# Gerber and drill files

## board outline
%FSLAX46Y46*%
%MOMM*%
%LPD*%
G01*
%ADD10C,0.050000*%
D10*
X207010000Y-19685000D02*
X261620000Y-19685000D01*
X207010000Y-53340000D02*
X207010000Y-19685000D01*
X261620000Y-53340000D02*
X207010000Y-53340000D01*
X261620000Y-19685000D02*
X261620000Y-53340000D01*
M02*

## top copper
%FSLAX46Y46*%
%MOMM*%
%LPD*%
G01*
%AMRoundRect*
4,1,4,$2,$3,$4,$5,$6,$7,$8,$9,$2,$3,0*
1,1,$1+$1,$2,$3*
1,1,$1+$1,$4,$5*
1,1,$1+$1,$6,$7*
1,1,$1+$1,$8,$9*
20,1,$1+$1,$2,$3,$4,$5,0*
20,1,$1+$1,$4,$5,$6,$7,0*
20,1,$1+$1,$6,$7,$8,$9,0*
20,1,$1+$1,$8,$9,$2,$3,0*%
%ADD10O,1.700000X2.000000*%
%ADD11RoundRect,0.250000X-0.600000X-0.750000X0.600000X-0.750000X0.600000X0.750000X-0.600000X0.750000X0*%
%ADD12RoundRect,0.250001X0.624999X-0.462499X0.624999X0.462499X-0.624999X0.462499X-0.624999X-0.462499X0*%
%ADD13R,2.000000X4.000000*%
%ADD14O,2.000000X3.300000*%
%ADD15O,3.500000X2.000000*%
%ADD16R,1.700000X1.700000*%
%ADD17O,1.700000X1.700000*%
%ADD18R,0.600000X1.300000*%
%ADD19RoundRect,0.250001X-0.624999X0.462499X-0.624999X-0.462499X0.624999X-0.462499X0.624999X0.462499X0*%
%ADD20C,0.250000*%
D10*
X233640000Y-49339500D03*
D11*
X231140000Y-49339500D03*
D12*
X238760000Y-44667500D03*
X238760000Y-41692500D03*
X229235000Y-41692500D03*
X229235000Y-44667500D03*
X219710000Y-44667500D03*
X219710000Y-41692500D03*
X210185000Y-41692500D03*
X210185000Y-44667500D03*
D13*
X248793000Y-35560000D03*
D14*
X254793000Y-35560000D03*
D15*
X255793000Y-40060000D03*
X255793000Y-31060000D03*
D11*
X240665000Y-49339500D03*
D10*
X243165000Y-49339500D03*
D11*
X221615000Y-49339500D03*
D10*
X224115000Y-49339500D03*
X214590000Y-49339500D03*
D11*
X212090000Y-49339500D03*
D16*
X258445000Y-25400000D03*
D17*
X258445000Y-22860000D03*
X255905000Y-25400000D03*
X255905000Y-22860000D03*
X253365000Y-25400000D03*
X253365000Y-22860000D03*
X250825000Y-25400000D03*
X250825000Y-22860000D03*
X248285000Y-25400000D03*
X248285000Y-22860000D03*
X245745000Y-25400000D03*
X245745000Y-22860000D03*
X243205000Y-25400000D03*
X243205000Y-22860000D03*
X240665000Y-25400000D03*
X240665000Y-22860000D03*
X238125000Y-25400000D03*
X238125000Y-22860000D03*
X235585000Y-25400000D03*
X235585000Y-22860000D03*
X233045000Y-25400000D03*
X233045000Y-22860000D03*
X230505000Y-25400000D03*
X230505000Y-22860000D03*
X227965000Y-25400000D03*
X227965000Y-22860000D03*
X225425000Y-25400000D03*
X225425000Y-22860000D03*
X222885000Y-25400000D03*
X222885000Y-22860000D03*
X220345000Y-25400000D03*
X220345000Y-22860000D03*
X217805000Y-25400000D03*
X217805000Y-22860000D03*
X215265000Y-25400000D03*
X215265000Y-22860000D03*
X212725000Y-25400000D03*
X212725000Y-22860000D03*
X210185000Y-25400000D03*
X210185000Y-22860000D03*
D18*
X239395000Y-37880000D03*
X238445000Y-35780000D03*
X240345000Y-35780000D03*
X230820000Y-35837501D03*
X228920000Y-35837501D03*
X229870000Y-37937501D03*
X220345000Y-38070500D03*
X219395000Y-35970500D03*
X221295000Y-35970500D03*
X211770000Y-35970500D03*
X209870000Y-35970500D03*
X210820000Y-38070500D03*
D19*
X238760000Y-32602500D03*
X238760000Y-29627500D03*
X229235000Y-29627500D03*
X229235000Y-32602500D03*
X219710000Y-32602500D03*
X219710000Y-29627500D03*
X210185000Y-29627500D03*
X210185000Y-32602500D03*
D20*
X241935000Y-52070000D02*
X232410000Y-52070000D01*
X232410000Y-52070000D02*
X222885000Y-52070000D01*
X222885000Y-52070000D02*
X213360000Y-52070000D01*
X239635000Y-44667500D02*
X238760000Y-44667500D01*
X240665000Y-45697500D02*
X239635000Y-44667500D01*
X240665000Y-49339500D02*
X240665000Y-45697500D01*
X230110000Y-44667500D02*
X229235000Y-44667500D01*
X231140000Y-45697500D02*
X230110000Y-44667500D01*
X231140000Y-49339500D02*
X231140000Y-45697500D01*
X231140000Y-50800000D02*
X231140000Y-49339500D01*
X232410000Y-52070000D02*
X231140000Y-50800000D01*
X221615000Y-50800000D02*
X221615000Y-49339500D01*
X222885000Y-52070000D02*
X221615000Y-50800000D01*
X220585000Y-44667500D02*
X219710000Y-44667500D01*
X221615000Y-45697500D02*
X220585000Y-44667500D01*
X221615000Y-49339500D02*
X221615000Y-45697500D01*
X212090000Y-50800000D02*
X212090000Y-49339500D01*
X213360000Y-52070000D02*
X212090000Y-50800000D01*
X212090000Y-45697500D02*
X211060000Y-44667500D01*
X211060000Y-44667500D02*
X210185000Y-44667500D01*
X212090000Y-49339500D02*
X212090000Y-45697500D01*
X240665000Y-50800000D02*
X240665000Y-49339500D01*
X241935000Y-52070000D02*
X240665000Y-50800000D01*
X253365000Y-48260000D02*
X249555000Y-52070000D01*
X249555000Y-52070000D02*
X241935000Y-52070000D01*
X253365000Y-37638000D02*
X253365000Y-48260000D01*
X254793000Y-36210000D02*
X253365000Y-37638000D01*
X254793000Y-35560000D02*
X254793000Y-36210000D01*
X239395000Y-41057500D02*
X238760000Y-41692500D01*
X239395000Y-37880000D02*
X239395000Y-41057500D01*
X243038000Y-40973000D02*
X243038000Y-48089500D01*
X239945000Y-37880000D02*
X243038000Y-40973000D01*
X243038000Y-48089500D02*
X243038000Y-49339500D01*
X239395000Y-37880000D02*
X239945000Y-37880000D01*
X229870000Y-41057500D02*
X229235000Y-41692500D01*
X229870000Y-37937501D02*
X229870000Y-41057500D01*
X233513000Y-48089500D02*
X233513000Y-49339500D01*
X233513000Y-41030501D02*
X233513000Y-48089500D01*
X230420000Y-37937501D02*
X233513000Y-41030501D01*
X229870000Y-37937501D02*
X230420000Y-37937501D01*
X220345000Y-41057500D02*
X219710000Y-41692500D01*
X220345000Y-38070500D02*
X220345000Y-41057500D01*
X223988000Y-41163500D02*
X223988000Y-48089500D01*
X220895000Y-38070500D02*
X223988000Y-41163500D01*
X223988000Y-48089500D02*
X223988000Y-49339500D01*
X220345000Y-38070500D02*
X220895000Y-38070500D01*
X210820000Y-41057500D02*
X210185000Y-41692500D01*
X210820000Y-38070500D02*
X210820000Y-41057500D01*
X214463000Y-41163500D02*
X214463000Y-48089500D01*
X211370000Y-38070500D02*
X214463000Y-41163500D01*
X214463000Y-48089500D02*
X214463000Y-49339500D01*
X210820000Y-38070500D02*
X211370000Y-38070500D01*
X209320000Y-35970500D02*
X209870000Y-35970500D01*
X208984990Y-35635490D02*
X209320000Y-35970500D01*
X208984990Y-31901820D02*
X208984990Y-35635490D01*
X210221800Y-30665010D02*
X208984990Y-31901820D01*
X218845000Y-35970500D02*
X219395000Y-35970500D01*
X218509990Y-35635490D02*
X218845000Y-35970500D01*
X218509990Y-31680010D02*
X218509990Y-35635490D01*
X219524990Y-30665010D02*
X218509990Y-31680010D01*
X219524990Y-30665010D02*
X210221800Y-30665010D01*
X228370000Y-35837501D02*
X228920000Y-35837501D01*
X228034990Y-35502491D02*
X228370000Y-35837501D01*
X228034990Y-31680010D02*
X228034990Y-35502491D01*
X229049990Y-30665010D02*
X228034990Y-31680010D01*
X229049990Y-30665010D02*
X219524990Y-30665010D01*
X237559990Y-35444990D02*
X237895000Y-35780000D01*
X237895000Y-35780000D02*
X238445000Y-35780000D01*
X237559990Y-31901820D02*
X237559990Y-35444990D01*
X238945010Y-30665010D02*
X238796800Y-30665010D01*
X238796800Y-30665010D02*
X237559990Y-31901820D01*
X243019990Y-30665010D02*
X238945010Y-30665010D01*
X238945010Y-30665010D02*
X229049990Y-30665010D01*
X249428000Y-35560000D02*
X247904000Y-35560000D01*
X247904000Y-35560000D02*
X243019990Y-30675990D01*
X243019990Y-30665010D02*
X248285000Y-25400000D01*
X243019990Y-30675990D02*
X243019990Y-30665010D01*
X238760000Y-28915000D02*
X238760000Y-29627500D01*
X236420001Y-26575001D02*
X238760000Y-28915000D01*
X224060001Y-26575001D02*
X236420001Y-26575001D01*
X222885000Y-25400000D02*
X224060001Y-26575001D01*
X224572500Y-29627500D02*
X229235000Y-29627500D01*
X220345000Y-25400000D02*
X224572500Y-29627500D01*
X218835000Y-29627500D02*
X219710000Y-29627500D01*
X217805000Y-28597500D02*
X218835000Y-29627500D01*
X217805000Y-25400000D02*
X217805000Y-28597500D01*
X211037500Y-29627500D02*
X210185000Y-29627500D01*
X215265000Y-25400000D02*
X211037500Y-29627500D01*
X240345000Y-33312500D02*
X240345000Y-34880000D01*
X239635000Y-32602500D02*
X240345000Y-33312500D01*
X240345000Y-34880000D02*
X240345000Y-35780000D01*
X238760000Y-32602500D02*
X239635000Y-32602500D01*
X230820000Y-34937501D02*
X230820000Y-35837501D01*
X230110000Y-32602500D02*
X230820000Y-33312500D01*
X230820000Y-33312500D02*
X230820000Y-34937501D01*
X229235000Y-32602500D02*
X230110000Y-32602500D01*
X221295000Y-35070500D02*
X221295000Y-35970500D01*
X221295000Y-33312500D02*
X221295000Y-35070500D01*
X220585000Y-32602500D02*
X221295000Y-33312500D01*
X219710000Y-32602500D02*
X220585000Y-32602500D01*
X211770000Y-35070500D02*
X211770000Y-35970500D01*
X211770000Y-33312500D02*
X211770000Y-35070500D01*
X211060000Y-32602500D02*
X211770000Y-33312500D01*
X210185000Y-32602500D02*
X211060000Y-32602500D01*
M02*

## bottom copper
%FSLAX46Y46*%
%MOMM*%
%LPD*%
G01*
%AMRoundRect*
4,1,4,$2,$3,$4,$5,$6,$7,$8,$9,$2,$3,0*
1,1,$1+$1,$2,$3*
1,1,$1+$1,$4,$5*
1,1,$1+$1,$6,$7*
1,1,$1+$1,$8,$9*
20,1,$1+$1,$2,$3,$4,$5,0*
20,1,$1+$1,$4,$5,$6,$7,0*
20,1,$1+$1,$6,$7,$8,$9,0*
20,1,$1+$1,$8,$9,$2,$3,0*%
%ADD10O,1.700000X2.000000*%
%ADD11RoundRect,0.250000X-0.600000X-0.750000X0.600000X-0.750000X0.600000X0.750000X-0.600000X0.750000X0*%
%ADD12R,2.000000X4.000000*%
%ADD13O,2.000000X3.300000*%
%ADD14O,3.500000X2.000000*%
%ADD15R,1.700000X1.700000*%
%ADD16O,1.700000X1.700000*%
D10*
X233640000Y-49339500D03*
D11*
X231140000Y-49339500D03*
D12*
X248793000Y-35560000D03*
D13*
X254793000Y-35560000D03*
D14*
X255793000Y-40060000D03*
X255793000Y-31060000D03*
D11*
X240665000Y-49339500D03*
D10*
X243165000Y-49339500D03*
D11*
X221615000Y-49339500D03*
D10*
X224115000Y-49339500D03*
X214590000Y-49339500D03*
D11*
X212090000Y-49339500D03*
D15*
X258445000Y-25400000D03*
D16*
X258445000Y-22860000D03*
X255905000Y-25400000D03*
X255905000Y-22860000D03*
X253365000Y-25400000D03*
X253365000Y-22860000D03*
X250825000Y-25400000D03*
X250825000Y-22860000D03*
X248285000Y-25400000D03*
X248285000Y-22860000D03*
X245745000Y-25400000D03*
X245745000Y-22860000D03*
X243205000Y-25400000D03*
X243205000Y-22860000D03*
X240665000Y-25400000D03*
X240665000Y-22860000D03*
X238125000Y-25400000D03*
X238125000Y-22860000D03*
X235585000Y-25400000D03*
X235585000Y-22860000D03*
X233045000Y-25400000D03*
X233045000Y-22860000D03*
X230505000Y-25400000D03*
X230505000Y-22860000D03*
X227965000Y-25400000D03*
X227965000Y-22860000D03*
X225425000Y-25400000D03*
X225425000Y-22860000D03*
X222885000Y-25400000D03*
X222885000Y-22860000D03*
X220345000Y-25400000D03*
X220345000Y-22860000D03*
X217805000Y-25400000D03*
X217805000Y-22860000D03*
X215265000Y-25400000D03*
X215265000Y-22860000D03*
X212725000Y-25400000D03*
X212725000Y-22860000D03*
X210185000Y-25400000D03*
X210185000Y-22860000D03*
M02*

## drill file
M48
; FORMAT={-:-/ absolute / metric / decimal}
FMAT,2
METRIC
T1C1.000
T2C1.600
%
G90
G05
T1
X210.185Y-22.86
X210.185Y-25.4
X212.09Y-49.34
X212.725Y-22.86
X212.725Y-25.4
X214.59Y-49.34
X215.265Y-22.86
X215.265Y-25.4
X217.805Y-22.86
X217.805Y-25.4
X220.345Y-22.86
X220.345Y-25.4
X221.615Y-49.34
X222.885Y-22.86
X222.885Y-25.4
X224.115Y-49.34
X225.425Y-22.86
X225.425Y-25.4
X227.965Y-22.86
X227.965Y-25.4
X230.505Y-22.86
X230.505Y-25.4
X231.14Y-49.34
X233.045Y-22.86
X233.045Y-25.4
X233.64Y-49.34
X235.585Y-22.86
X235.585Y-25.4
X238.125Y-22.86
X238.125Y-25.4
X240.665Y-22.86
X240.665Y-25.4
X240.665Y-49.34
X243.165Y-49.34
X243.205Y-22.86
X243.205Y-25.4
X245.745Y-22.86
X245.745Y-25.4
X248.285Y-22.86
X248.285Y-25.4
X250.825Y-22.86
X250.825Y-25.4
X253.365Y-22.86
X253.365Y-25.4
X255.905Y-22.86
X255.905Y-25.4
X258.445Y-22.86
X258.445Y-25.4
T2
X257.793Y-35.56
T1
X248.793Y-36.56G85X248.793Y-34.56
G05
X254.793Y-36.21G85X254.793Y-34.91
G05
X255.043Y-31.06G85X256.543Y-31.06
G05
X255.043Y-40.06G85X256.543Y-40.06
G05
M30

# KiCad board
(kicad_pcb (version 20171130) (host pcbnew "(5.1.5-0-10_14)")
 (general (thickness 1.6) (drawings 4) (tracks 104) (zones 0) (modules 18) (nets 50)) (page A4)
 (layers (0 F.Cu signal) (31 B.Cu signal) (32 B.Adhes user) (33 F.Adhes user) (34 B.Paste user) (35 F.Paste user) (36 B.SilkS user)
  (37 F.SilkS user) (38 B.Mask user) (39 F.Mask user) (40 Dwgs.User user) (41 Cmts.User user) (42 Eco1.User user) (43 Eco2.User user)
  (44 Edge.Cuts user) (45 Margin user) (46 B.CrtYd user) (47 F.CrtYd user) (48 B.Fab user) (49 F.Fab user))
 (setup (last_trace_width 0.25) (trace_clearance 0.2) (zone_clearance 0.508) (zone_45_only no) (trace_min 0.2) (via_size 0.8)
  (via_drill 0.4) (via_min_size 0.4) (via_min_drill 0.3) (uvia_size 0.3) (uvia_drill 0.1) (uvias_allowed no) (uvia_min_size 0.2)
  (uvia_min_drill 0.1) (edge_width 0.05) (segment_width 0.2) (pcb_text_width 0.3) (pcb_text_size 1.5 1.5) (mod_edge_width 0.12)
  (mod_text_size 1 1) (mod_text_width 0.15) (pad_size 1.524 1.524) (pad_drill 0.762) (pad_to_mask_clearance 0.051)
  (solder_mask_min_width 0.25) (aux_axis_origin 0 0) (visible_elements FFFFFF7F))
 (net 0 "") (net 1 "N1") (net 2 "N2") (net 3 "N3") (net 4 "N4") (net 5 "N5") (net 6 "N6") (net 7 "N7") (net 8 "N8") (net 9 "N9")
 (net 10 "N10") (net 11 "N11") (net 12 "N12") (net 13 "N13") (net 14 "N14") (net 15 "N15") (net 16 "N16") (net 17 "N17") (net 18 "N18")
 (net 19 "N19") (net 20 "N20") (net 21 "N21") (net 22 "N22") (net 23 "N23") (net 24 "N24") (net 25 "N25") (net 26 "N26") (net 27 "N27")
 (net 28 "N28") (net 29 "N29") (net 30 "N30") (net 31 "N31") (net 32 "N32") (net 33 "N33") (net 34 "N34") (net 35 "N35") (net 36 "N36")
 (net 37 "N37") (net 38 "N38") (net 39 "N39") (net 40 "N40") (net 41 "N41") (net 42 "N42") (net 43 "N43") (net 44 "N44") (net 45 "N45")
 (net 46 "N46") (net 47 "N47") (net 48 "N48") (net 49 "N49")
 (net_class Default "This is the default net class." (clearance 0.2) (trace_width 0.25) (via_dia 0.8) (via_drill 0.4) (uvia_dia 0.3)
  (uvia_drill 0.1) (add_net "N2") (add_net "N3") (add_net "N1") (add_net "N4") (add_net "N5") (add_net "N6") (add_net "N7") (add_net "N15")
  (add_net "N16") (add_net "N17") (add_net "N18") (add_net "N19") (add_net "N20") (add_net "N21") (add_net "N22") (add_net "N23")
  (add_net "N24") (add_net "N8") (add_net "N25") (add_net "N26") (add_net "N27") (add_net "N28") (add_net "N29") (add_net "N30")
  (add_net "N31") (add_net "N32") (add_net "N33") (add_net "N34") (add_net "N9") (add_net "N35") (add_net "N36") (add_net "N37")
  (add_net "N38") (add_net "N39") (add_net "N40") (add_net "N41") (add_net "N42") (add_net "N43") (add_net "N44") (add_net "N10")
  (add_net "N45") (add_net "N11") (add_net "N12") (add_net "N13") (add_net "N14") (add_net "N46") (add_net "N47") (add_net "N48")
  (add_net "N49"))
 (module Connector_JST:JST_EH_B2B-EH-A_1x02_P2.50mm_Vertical (layer F.Cu) (at 231.14 49.3395)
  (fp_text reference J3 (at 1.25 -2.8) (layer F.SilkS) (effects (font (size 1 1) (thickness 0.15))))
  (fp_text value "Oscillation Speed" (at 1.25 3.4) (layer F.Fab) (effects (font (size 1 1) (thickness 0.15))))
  (pad 2 thru_hole oval (at 2.5 0) (size 1.7 2) (drill 1) (layers *.Cu *.Mask) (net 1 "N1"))
  (pad 1 thru_hole roundrect (at 0 0) (size 1.7 2) (drill 1) (layers *.Cu *.Mask) (roundrect_rratio 0.147059) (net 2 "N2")))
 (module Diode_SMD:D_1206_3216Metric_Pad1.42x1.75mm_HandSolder (layer F.Cu) (at 238.76 43.18 90)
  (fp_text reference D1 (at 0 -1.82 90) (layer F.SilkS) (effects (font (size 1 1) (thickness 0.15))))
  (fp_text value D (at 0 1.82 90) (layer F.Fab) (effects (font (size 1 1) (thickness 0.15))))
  (pad 1 smd roundrect (at -1.4875 0 90) (size 1.425 1.75) (layers F.Cu F.Paste F.Mask) (roundrect_rratio 0.175439) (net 2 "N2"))
  (pad 2 smd roundrect (at 1.4875 0 90) (size 1.425 1.75) (layers F.Cu F.Paste F.Mask) (roundrect_rratio 0.175439) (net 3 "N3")))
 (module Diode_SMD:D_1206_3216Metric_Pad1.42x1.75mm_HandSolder (layer F.Cu) (at 229.235 43.18 90)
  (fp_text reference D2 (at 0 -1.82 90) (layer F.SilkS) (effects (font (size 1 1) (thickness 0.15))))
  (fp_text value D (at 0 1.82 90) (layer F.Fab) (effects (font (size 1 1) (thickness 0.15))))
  (pad 2 smd roundrect (at 1.4875 0 90) (size 1.425 1.75) (layers F.Cu F.Paste F.Mask) (roundrect_rratio 0.175439) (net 1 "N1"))
  (pad 1 smd roundrect (at -1.4875 0 90) (size 1.425 1.75) (layers F.Cu F.Paste F.Mask) (roundrect_rratio 0.175439) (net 2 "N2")))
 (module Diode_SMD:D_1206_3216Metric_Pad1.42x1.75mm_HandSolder (layer F.Cu) (at 219.71 43.18 90)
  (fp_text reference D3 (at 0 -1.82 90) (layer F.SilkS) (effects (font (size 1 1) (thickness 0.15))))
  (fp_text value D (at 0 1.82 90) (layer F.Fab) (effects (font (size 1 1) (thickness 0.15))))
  (pad 1 smd roundrect (at -1.4875 0 90) (size 1.425 1.75) (layers F.Cu F.Paste F.Mask) (roundrect_rratio 0.175439) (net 2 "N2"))
  (pad 2 smd roundrect (at 1.4875 0 90) (size 1.425 1.75) (layers F.Cu F.Paste F.Mask) (roundrect_rratio 0.175439) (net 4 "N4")))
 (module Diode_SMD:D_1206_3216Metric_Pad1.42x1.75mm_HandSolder (layer F.Cu) (at 210.185 43.18 90)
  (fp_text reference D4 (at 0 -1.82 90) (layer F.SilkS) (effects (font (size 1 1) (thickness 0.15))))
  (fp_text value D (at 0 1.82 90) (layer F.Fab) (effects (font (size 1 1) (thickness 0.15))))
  (pad 2 smd roundrect (at 1.4875 0 90) (size 1.425 1.75) (layers F.Cu F.Paste F.Mask) (roundrect_rratio 0.175439) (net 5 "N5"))
  (pad 1 smd roundrect (at -1.4875 0 90) (size 1.425 1.75) (layers F.Cu F.Paste F.Mask) (roundrect_rratio 0.175439) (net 2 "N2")))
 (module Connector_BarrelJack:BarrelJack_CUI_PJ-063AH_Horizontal (layer F.Cu) (at 248.793 35.56 90)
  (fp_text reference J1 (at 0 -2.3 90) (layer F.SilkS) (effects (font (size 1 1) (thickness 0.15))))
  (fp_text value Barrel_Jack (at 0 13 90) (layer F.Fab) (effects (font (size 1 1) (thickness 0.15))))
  (pad 1 thru_hole rect (at 0 0 90) (size 4 2) (drill oval 3 1) (layers *.Cu *.Mask) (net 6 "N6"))
  (pad 2 thru_hole oval (at 0 6 90) (size 3.3 2) (drill oval 2.3 1) (layers *.Cu *.Mask) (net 2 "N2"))
  (pad MP thru_hole oval (at -4.5 7 90) (size 2 3.5) (drill oval 1 2.5) (layers *.Cu *.Mask))
  (pad MP thru_hole oval (at 4.5 7 90) (size 2 3.5) (drill oval 1 2.5) (layers *.Cu *.Mask))
  (pad "" np_thru_hole circle (at 0 9 90) (size 1.6 1.6) (drill 1.6) (layers *.Cu *.Mask)))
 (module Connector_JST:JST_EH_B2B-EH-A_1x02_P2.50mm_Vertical (layer F.Cu) (at 240.665 49.3395)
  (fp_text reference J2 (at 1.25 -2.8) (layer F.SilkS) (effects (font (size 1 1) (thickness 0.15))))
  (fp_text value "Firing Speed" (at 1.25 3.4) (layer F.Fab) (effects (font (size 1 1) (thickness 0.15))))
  (pad 1 thru_hole roundrect (at 0 0) (size 1.7 2) (drill 1) (layers *.Cu *.Mask) (roundrect_rratio 0.147059) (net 2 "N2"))
  (pad 2 thru_hole oval (at 2.5 0) (size 1.7 2) (drill 1) (layers *.Cu *.Mask) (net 3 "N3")))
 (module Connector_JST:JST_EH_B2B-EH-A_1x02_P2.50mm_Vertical (layer F.Cu) (at 221.615 49.3395)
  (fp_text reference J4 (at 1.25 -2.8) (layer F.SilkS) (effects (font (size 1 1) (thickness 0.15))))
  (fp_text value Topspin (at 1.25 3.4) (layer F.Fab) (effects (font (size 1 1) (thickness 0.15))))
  (pad 1 thru_hole roundrect (at 0 0) (size 1.7 2) (drill 1) (layers *.Cu *.Mask) (roundrect_rratio 0.147059) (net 2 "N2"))
  (pad 2 thru_hole oval (at 2.5 0) (size 1.7 2) (drill 1) (layers *.Cu *.Mask) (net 4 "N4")))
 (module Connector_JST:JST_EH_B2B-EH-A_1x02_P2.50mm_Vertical (layer F.Cu) (at 212.09 49.3395)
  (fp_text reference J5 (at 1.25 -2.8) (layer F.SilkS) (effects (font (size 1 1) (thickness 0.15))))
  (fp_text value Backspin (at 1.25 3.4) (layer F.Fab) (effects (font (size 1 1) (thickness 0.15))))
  (pad 2 thru_hole oval (at 2.5 0) (size 1.7 2) (drill 1) (layers *.Cu *.Mask) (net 5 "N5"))
  (pad 1 thru_hole roundrect (at 0 0) (size 1.7 2) (drill 1) (layers *.Cu *.Mask) (roundrect_rratio 0.147059) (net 2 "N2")))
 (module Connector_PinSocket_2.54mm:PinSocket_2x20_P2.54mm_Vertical (layer F.Cu) (at 258.445 25.4 270)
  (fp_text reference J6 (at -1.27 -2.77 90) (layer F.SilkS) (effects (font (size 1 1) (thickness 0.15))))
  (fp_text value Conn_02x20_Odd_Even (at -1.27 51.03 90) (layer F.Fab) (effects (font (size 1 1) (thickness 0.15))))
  (pad 1 thru_hole rect (at 0 0 270) (size 1.7 1.7) (drill 1) (layers *.Cu *.Mask) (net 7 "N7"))
  (pad 2 thru_hole oval (at -2.54 0 270) (size 1.7 1.7) (drill 1) (layers *.Cu *.Mask) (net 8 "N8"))
  (pad 3 thru_hole oval (at 0 2.54 270) (size 1.7 1.7) (drill 1) (layers *.Cu *.Mask) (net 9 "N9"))
  (pad 4 thru_hole oval (at -2.54 2.54 270) (size 1.7 1.7) (drill 1) (layers *.Cu *.Mask) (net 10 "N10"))
  (pad 5 thru_hole oval (at 0 5.08 270) (size 1.7 1.7) (drill 1) (layers *.Cu *.Mask) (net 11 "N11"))
  (pad 6 thru_hole oval (at -2.54 5.08 270) (size 1.7 1.7) (drill 1) (layers *.Cu *.Mask) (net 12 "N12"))
  (pad 7 thru_hole oval (at 0 7.62 270) (size 1.7 1.7) (drill 1) (layers *.Cu *.Mask) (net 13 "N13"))
  (pad 8 thru_hole oval (at -2.54 7.62 270) (size 1.7 1.7) (drill 1) (layers *.Cu *.Mask) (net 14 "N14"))
  (pad 9 thru_hole oval (at 0 10.16 270) (size 1.7 1.7) (drill 1) (layers *.Cu *.Mask) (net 6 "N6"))
  (pad 10 thru_hole oval (at -2.54 10.16 270) (size 1.7 1.7) (drill 1) (layers *.Cu *.Mask) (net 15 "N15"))
  (pad 11 thru_hole oval (at 0 12.7 270) (size 1.7 1.7) (drill 1) (layers *.Cu *.Mask) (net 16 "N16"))
  (pad 12 thru_hole oval (at -2.54 12.7 270) (size 1.7 1.7) (drill 1) (layers *.Cu *.Mask) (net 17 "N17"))
  (pad 13 thru_hole oval (at 0 15.24 270) (size 1.7 1.7) (drill 1) (layers *.Cu *.Mask) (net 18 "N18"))
  (pad 14 thru_hole oval (at -2.54 15.24 270) (size 1.7 1.7) (drill 1) (layers *.Cu *.Mask) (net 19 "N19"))
  (pad 15 thru_hole oval (at 0 17.78 270) (size 1.7 1.7) (drill 1) (layers *.Cu *.Mask) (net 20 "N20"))
  (pad 16 thru_hole oval (at -2.54 17.78 270) (size 1.7 1.7) (drill 1) (layers *.Cu *.Mask) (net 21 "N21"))
  (pad 17 thru_hole oval (at 0 20.32 270) (size 1.7 1.7) (drill 1) (layers *.Cu *.Mask) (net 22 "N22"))
  (pad 18 thru_hole oval (at -2.54 20.32 270) (size 1.7 1.7) (drill 1) (layers *.Cu *.Mask) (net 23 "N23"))
  (pad 19 thru_hole oval (at 0 22.86 270) (size 1.7 1.7) (drill 1) (layers *.Cu *.Mask) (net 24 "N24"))
  (pad 20 thru_hole oval (at -2.54 22.86 270) (size 1.7 1.7) (drill 1) (layers *.Cu *.Mask) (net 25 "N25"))
  (pad 21 thru_hole oval (at 0 25.4 270) (size 1.7 1.7) (drill 1) (layers *.Cu *.Mask) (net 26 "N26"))
  (pad 22 thru_hole oval (at -2.54 25.4 270) (size 1.7 1.7) (drill 1) (layers *.Cu *.Mask) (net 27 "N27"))
  (pad 23 thru_hole oval (at 0 27.94 270) (size 1.7 1.7) (drill 1) (layers *.Cu *.Mask) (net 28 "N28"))
  (pad 24 thru_hole oval (at -2.54 27.94 270) (size 1.7 1.7) (drill 1) (layers *.Cu *.Mask) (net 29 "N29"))
  (pad 25 thru_hole oval (at 0 30.48 270) (size 1.7 1.7) (drill 1) (layers *.Cu *.Mask) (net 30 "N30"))
  (pad 26 thru_hole oval (at -2.54 30.48 270) (size 1.7 1.7) (drill 1) (layers *.Cu *.Mask) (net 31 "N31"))
  (pad 27 thru_hole oval (at 0 33.02 270) (size 1.7 1.7) (drill 1) (layers *.Cu *.Mask) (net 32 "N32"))
  (pad 28 thru_hole oval (at -2.54 33.02 270) (size 1.7 1.7) (drill 1) (layers *.Cu *.Mask) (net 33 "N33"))
  (pad 29 thru_hole oval (at 0 35.56 270) (size 1.7 1.7) (drill 1) (layers *.Cu *.Mask) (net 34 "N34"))
  (pad 30 thru_hole oval (at -2.54 35.56 270) (size 1.7 1.7) (drill 1) (layers *.Cu *.Mask) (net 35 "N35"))
  (pad 31 thru_hole oval (at 0 38.1 270) (size 1.7 1.7) (drill 1) (layers *.Cu *.Mask) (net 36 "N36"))
  (pad 32 thru_hole oval (at -2.54 38.1 270) (size 1.7 1.7) (drill 1) (layers *.Cu *.Mask) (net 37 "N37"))
  (pad 33 thru_hole oval (at 0 40.64 270) (size 1.7 1.7) (drill 1) (layers *.Cu *.Mask) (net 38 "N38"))
  (pad 34 thru_hole oval (at -2.54 40.64 270) (size 1.7 1.7) (drill 1) (layers *.Cu *.Mask) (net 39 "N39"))
  (pad 35 thru_hole oval (at 0 43.18 270) (size 1.7 1.7) (drill 1) (layers *.Cu *.Mask) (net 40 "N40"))
  (pad 36 thru_hole oval (at -2.54 43.18 270) (size 1.7 1.7) (drill 1) (layers *.Cu *.Mask) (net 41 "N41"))
  (pad 37 thru_hole oval (at 0 45.72 270) (size 1.7 1.7) (drill 1) (layers *.Cu *.Mask) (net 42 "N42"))
  (pad 38 thru_hole oval (at -2.54 45.72 270) (size 1.7 1.7) (drill 1) (layers *.Cu *.Mask) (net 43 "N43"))
  (pad 39 thru_hole oval (at 0 48.26 270) (size 1.7 1.7) (drill 1) (layers *.Cu *.Mask) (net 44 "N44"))
  (pad 40 thru_hole oval (at -2.54 48.26 270) (size 1.7 1.7) (drill 1) (layers *.Cu *.Mask) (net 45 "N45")))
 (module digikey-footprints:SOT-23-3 (layer F.Cu) (at 239.395 36.83 270)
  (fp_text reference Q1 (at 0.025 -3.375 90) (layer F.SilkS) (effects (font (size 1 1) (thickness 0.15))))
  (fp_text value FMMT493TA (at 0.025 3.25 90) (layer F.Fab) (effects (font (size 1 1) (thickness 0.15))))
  (pad 3 smd rect (at 1.05 0 270) (size 1.3 0.6) (layers F.Cu F.Paste F.Mask) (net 3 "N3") (solder_mask_margin 0.07))
  (pad 2 smd rect (at -1.05 0.95 270) (size 1.3 0.6) (layers F.Cu F.Paste F.Mask) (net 6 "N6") (solder_mask_margin 0.07))
  (pad 1 smd rect (at -1.05 -0.95 270) (size 1.3 0.6) (layers F.Cu F.Paste F.Mask) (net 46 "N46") (solder_mask_margin 0.07)))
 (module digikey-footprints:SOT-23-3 (layer F.Cu) (at 229.87 36.887501 270)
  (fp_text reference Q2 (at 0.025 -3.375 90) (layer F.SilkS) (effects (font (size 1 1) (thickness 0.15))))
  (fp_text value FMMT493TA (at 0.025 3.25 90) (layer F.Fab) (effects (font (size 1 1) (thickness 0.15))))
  (pad 1 smd rect (at -1.05 -0.95 270) (size 1.3 0.6) (layers F.Cu F.Paste F.Mask) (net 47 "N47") (solder_mask_margin 0.07))
  (pad 2 smd rect (at -1.05 0.95 270) (size 1.3 0.6) (layers F.Cu F.Paste F.Mask) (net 6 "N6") (solder_mask_margin 0.07))
  (pad 3 smd rect (at 1.05 0 270) (size 1.3 0.6) (layers F.Cu F.Paste F.Mask) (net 1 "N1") (solder_mask_margin 0.07)))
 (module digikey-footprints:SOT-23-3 (layer F.Cu) (at 220.345 37.0205 270)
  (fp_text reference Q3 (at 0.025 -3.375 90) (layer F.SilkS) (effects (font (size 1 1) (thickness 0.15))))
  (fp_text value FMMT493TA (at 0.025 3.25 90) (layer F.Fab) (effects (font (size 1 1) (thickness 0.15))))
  (pad 3 smd rect (at 1.05 0 270) (size 1.3 0.6) (layers F.Cu F.Paste F.Mask) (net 4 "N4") (solder_mask_margin 0.07))
  (pad 2 smd rect (at -1.05 0.95 270) (size 1.3 0.6) (layers F.Cu F.Paste F.Mask) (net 6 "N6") (solder_mask_margin 0.07))
  (pad 1 smd rect (at -1.05 -0.95 270) (size 1.3 0.6) (layers F.Cu F.Paste F.Mask) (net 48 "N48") (solder_mask_margin 0.07)))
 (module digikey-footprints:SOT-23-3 (layer F.Cu) (at 210.82 37.0205 270)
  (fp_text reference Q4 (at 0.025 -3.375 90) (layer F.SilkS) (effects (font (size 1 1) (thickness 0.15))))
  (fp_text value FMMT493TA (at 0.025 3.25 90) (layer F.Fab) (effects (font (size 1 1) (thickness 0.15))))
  (pad 1 smd rect (at -1.05 -0.95 270) (size 1.3 0.6) (layers F.Cu F.Paste F.Mask) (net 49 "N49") (solder_mask_margin 0.07))
  (pad 2 smd rect (at -1.05 0.95 270) (size 1.3 0.6) (layers F.Cu F.Paste F.Mask) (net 6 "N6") (solder_mask_margin 0.07))
  (pad 3 smd rect (at 1.05 0 270) (size 1.3 0.6) (layers F.Cu F.Paste F.Mask) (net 5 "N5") (solder_mask_margin 0.07)))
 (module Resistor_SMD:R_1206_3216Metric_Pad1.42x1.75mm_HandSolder (layer F.Cu) (at 238.76 31.115 270)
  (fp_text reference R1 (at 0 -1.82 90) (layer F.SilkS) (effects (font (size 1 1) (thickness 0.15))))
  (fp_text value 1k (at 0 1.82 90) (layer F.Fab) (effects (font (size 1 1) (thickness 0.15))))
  (pad 2 smd roundrect (at 1.4875 0 270) (size 1.425 1.75) (layers F.Cu F.Paste F.Mask) (roundrect_rratio 0.175439) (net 46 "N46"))
  (pad 1 smd roundrect (at -1.4875 0 270) (size 1.425 1.75) (layers F.Cu F.Paste F.Mask) (roundrect_rratio 0.175439) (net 34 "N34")))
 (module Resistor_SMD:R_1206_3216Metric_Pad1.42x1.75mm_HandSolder (layer F.Cu) (at 229.235 31.115 270)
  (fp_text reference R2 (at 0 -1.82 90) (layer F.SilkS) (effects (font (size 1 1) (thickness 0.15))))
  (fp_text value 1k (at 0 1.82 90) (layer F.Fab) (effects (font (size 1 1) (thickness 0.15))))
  (pad 1 smd roundrect (at -1.4875 0 270) (size 1.425 1.75) (layers F.Cu F.Paste F.Mask) (roundrect_rratio 0.175439) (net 36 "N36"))
  (pad 2 smd roundrect (at 1.4875 0 270) (size 1.425 1.75) (layers F.Cu F.Paste F.Mask) (roundrect_rratio 0.175439) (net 47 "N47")))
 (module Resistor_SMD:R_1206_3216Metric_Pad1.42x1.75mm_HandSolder (layer F.Cu) (at 219.71 31.115 270)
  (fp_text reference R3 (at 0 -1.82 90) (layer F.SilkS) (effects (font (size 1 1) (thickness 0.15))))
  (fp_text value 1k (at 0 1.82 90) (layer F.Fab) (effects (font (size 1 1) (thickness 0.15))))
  (pad 2 smd roundrect (at 1.4875 0 270) (size 1.425 1.75) (layers F.Cu F.Paste F.Mask) (roundrect_rratio 0.175439) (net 48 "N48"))
  (pad 1 smd roundrect (at -1.4875 0 270) (size 1.425 1.75) (layers F.Cu F.Paste F.Mask) (roundrect_rratio 0.175439) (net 38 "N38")))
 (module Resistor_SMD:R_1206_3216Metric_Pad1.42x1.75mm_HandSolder (layer F.Cu) (at 210.185 31.115 270)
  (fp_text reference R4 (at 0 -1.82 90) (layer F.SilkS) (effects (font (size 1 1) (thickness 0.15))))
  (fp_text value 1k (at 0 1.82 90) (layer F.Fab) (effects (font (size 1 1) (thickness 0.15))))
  (pad 1 smd roundrect (at -1.4875 0 270) (size 1.425 1.75) (layers F.Cu F.Paste F.Mask) (roundrect_rratio 0.175439) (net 40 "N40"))
  (pad 2 smd roundrect (at 1.4875 0 270) (size 1.425 1.75) (layers F.Cu F.Paste F.Mask) (roundrect_rratio 0.175439) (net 49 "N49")))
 (gr_line (start 207.01 19.685) (end 261.62 19.685) (layer Edge.Cuts) (width 0.05))
 (gr_line (start 207.01 53.34) (end 207.01 19.685) (layer Edge.Cuts) (width 0.05))
 (gr_line (start 261.62 53.34) (end 207.01 53.34) (layer Edge.Cuts) (width 0.05))
 (gr_line (start 261.62 19.685) (end 261.62 53.34) (layer Edge.Cuts) (width 0.05))
 (segment (start 241.935 52.07) (end 232.41 52.07) (width 0.25) (layer F.Cu) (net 2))
 (segment (start 232.41 52.07) (end 222.885 52.07) (width 0.25) (layer F.Cu) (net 2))
 (segment (start 222.885 52.07) (end 213.36 52.07) (width 0.25) (layer F.Cu) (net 2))
 (segment (start 239.635 44.6675) (end 238.76 44.6675) (width 0.25) (layer F.Cu) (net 2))
 (segment (start 240.665 45.6975) (end 239.635 44.6675) (width 0.25) (layer F.Cu) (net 2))
 (segment (start 240.665 49.3395) (end 240.665 45.6975) (width 0.25) (layer F.Cu) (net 2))
 (segment (start 230.11 44.6675) (end 229.235 44.6675) (width 0.25) (layer F.Cu) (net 2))
 (segment (start 231.14 45.6975) (end 230.11 44.6675) (width 0.25) (layer F.Cu) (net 2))
 (segment (start 231.14 49.3395) (end 231.14 45.6975) (width 0.25) (layer F.Cu) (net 2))
 (segment (start 231.14 50.8) (end 231.14 49.3395) (width 0.25) (layer F.Cu) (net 2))
 (segment (start 232.41 52.07) (end 231.14 50.8) (width 0.25) (layer F.Cu) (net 2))
 (segment (start 221.615 50.8) (end 221.615 49.3395) (width 0.25) (layer F.Cu) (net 2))
 (segment (start 222.885 52.07) (end 221.615 50.8) (width 0.25) (layer F.Cu) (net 2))
 (segment (start 220.585 44.6675) (end 219.71 44.6675) (width 0.25) (layer F.Cu) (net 2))
 (segment (start 221.615 45.6975) (end 220.585 44.6675) (width 0.25) (layer F.Cu) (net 2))
 (segment (start 221.615 49.3395) (end 221.615 45.6975) (width 0.25) (layer F.Cu) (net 2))
 (segment (start 212.09 50.8) (end 212.09 49.3395) (width 0.25) (layer F.Cu) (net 2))
 (segment (start 213.36 52.07) (end 212.09 50.8) (width 0.25) (layer F.Cu) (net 2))
 (segment (start 212.09 45.6975) (end 211.06 44.6675) (width 0.25) (layer F.Cu) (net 2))
 (segment (start 211.06 44.6675) (end 210.185 44.6675) (width 0.25) (layer F.Cu) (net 2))
 (segment (start 212.09 49.3395) (end 212.09 45.6975) (width 0.25) (layer F.Cu) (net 2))
 (segment (start 240.665 50.8) (end 240.665 49.3395) (width 0.25) (layer F.Cu) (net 2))
 (segment (start 241.935 52.07) (end 240.665 50.8) (width 0.25) (layer F.Cu) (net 2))
 (segment (start 253.365 48.26) (end 249.555 52.07) (width 0.25) (layer F.Cu) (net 2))
 (segment (start 249.555 52.07) (end 241.935 52.07) (width 0.25) (layer F.Cu) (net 2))
 (segment (start 253.365 37.638) (end 253.365 48.26) (width 0.25) (layer F.Cu) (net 2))
 (segment (start 254.793 36.21) (end 253.365 37.638) (width 0.25) (layer F.Cu) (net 2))
 (segment (start 254.793 35.56) (end 254.793 36.21) (width 0.25) (layer F.Cu) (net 2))
 (segment (start 239.395 41.0575) (end 238.76 41.6925) (width 0.25) (layer F.Cu) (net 3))
 (segment (start 239.395 37.88) (end 239.395 41.0575) (width 0.25) (layer F.Cu) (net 3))
 (segment (start 243.038 40.973) (end 243.038 48.0895) (width 0.25) (layer F.Cu) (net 3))
 (segment (start 239.945 37.88) (end 243.038 40.973) (width 0.25) (layer F.Cu) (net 3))
 (segment (start 243.038 48.0895) (end 243.038 49.3395) (width 0.25) (layer F.Cu) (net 3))
 (segment (start 239.395 37.88) (end 239.945 37.88) (width 0.25) (layer F.Cu) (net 3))
 (segment (start 229.87 41.0575) (end 229.235 41.6925) (width 0.25) (layer F.Cu) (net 1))
 (segment (start 229.87 37.937501) (end 229.87 41.0575) (width 0.25) (layer F.Cu) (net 1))
 (segment (start 233.513 48.0895) (end 233.513 49.3395) (width 0.25) (layer F.Cu) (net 1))
 (segment (start 233.513 41.030501) (end 233.513 48.0895) (width 0.25) (layer F.Cu) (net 1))
 (segment (start 230.42 37.937501) (end 233.513 41.030501) (width 0.25) (layer F.Cu) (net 1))
 (segment (start 229.87 37.937501) (end 230.42 37.937501) (width 0.25) (layer F.Cu) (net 1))
 (segment (start 220.345 41.0575) (end 219.71 41.6925) (width 0.25) (layer F.Cu) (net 4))
 (segment (start 220.345 38.0705) (end 220.345 41.0575) (width 0.25) (layer F.Cu) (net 4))
 (segment (start 223.988 41.1635) (end 223.988 48.0895) (width 0.25) (layer F.Cu) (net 4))
 (segment (start 220.895 38.0705) (end 223.988 41.1635) (width 0.25) (layer F.Cu) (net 4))
 (segment (start 223.988 48.0895) (end 223.988 49.3395) (width 0.25) (layer F.Cu) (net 4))
 (segment (start 220.345 38.0705) (end 220.895 38.0705) (width 0.25) (layer F.Cu) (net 4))
 (segment (start 210.82 41.0575) (end 210.185 41.6925) (width 0.25) (layer F.Cu) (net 5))
 (segment (start 210.82 38.0705) (end 210.82 41.0575) (width 0.25) (layer F.Cu) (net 5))
 (segment (start 214.463 41.1635) (end 214.463 48.0895) (width 0.25) (layer F.Cu) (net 5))
 (segment (start 211.37 38.0705) (end 214.463 41.1635) (width 0.25) (layer F.Cu) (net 5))
 (segment (start 214.463 48.0895) (end 214.463 49.3395) (width 0.25) (layer F.Cu) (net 5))
 (segment (start 210.82 38.0705) (end 211.37 38.0705) (width 0.25) (layer F.Cu) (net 5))
 (segment (start 209.32 35.9705) (end 209.87 35.9705) (width 0.25) (layer F.Cu) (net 6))
 (segment (start 208.98499 35.63549) (end 209.32 35.9705) (width 0.25) (layer F.Cu) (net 6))
 (segment (start 208.98499 31.90182) (end 208.98499 35.63549) (width 0.25) (layer F.Cu) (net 6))
 (segment (start 210.2218 30.66501) (end 208.98499 31.90182) (width 0.25) (layer F.Cu) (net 6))
 (segment (start 218.845 35.9705) (end 219.395 35.9705) (width 0.25) (layer F.Cu) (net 6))
 (segment (start 218.50999 35.63549) (end 218.845 35.9705) (width 0.25) (layer F.Cu) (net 6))
 (segment (start 218.50999 31.68001) (end 218.50999 35.63549) (width 0.25) (layer F.Cu) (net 6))
 (segment (start 219.52499 30.66501) (end 218.50999 31.68001) (width 0.25) (layer F.Cu) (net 6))
 (segment (start 219.52499 30.66501) (end 210.2218 30.66501) (width 0.25) (layer F.Cu) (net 6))
 (segment (start 228.37 35.837501) (end 228.92 35.837501) (width 0.25) (layer F.Cu) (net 6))
 (segment (start 228.03499 35.502491) (end 228.37 35.837501) (width 0.25) (layer F.Cu) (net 6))
 (segment (start 228.03499 31.68001) (end 228.03499 35.502491) (width 0.25) (layer F.Cu) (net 6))
 (segment (start 229.04999 30.66501) (end 228.03499 31.68001) (width 0.25) (layer F.Cu) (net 6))
 (segment (start 229.04999 30.66501) (end 219.52499 30.66501) (width 0.25) (layer F.Cu) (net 6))
 (segment (start 237.55999 35.44499) (end 237.895 35.78) (width 0.25) (layer F.Cu) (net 6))
 (segment (start 237.895 35.78) (end 238.445 35.78) (width 0.25) (layer F.Cu) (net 6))
 (segment (start 237.55999 31.90182) (end 237.55999 35.44499) (width 0.25) (layer F.Cu) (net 6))
 (segment (start 238.94501 30.66501) (end 238.7968 30.66501) (width 0.25) (layer F.Cu) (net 6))
 (segment (start 238.7968 30.66501) (end 237.55999 31.90182) (width 0.25) (layer F.Cu) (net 6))
 (segment (start 243.01999 30.66501) (end 238.94501 30.66501) (width 0.25) (layer F.Cu) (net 6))
 (segment (start 238.94501 30.66501) (end 229.04999 30.66501) (width 0.25) (layer F.Cu) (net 6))
 (segment (start 249.428 35.56) (end 247.904 35.56) (width 0.25) (layer F.Cu) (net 6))
 (segment (start 247.904 35.56) (end 243.01999 30.67599) (width 0.25) (layer F.Cu) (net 6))
 (segment (start 243.01999 30.66501) (end 248.285 25.4) (width 0.25) (layer F.Cu) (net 6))
 (segment (start 243.01999 30.67599) (end 243.01999 30.66501) (width 0.25) (layer F.Cu) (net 6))
 (segment (start 238.76 28.915) (end 238.76 29.6275) (width 0.25) (layer F.Cu) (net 34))
 (segment (start 236.420001 26.575001) (end 238.76 28.915) (width 0.25) (layer F.Cu) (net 34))
 (segment (start 224.060001 26.575001) (end 236.420001 26.575001) (width 0.25) (layer F.Cu) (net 34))
 (segment (start 222.885 25.4) (end 224.060001 26.575001) (width 0.25) (layer F.Cu) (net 34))
 (segment (start 224.5725 29.6275) (end 229.235 29.6275) (width 0.25) (layer F.Cu) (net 36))
 (segment (start 220.345 25.4) (end 224.5725 29.6275) (width 0.25) (layer F.Cu) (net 36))
 (segment (start 218.835 29.6275) (end 219.71 29.6275) (width 0.25) (layer F.Cu) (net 38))
 (segment (start 217.805 28.5975) (end 218.835 29.6275) (width 0.25) (layer F.Cu) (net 38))
 (segment (start 217.805 25.4) (end 217.805 28.5975) (width 0.25) (layer F.Cu) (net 38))
 (segment (start 211.0375 29.6275) (end 210.185 29.6275) (width 0.25) (layer F.Cu) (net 40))
 (segment (start 215.265 25.4) (end 211.0375 29.6275) (width 0.25) (layer F.Cu) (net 40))
 (segment (start 240.345 33.3125) (end 240.345 34.88) (width 0.25) (layer F.Cu) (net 46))
 (segment (start 239.635 32.6025) (end 240.345 33.3125) (width 0.25) (layer F.Cu) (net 46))
 (segment (start 240.345 34.88) (end 240.345 35.78) (width 0.25) (layer F.Cu) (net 46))
 (segment (start 238.76 32.6025) (end 239.635 32.6025) (width 0.25) (layer F.Cu) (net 46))
 (segment (start 230.82 34.937501) (end 230.82 35.837501) (width 0.25) (layer F.Cu) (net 47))
 (segment (start 230.11 32.6025) (end 230.82 33.3125) (width 0.25) (layer F.Cu) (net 47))
 (segment (start 230.82 33.3125) (end 230.82 34.937501) (width 0.25) (layer F.Cu) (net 47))
 (segment (start 229.235 32.6025) (end 230.11 32.6025) (width 0.25) (layer F.Cu) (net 47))
 (segment (start 221.295 35.0705) (end 221.295 35.9705) (width 0.25) (layer F.Cu) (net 48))
 (segment (start 221.295 33.3125) (end 221.295 35.0705) (width 0.25) (layer F.Cu) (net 48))
 (segment (start 220.585 32.6025) (end 221.295 33.3125) (width 0.25) (layer F.Cu) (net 48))
 (segment (start 219.71 32.6025) (end 220.585 32.6025) (width 0.25) (layer F.Cu) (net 48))
 (segment (start 211.77 35.0705) (end 211.77 35.9705) (width 0.25) (layer F.Cu) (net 49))
 (segment (start 211.77 33.3125) (end 211.77 35.0705) (width 0.25) (layer F.Cu) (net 49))
 (segment (start 211.06 32.6025) (end 211.77 33.3125) (width 0.25) (layer F.Cu) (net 49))
 (segment (start 210.185 32.6025) (end 211.06 32.6025) (width 0.25) (layer F.Cu) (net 49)))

